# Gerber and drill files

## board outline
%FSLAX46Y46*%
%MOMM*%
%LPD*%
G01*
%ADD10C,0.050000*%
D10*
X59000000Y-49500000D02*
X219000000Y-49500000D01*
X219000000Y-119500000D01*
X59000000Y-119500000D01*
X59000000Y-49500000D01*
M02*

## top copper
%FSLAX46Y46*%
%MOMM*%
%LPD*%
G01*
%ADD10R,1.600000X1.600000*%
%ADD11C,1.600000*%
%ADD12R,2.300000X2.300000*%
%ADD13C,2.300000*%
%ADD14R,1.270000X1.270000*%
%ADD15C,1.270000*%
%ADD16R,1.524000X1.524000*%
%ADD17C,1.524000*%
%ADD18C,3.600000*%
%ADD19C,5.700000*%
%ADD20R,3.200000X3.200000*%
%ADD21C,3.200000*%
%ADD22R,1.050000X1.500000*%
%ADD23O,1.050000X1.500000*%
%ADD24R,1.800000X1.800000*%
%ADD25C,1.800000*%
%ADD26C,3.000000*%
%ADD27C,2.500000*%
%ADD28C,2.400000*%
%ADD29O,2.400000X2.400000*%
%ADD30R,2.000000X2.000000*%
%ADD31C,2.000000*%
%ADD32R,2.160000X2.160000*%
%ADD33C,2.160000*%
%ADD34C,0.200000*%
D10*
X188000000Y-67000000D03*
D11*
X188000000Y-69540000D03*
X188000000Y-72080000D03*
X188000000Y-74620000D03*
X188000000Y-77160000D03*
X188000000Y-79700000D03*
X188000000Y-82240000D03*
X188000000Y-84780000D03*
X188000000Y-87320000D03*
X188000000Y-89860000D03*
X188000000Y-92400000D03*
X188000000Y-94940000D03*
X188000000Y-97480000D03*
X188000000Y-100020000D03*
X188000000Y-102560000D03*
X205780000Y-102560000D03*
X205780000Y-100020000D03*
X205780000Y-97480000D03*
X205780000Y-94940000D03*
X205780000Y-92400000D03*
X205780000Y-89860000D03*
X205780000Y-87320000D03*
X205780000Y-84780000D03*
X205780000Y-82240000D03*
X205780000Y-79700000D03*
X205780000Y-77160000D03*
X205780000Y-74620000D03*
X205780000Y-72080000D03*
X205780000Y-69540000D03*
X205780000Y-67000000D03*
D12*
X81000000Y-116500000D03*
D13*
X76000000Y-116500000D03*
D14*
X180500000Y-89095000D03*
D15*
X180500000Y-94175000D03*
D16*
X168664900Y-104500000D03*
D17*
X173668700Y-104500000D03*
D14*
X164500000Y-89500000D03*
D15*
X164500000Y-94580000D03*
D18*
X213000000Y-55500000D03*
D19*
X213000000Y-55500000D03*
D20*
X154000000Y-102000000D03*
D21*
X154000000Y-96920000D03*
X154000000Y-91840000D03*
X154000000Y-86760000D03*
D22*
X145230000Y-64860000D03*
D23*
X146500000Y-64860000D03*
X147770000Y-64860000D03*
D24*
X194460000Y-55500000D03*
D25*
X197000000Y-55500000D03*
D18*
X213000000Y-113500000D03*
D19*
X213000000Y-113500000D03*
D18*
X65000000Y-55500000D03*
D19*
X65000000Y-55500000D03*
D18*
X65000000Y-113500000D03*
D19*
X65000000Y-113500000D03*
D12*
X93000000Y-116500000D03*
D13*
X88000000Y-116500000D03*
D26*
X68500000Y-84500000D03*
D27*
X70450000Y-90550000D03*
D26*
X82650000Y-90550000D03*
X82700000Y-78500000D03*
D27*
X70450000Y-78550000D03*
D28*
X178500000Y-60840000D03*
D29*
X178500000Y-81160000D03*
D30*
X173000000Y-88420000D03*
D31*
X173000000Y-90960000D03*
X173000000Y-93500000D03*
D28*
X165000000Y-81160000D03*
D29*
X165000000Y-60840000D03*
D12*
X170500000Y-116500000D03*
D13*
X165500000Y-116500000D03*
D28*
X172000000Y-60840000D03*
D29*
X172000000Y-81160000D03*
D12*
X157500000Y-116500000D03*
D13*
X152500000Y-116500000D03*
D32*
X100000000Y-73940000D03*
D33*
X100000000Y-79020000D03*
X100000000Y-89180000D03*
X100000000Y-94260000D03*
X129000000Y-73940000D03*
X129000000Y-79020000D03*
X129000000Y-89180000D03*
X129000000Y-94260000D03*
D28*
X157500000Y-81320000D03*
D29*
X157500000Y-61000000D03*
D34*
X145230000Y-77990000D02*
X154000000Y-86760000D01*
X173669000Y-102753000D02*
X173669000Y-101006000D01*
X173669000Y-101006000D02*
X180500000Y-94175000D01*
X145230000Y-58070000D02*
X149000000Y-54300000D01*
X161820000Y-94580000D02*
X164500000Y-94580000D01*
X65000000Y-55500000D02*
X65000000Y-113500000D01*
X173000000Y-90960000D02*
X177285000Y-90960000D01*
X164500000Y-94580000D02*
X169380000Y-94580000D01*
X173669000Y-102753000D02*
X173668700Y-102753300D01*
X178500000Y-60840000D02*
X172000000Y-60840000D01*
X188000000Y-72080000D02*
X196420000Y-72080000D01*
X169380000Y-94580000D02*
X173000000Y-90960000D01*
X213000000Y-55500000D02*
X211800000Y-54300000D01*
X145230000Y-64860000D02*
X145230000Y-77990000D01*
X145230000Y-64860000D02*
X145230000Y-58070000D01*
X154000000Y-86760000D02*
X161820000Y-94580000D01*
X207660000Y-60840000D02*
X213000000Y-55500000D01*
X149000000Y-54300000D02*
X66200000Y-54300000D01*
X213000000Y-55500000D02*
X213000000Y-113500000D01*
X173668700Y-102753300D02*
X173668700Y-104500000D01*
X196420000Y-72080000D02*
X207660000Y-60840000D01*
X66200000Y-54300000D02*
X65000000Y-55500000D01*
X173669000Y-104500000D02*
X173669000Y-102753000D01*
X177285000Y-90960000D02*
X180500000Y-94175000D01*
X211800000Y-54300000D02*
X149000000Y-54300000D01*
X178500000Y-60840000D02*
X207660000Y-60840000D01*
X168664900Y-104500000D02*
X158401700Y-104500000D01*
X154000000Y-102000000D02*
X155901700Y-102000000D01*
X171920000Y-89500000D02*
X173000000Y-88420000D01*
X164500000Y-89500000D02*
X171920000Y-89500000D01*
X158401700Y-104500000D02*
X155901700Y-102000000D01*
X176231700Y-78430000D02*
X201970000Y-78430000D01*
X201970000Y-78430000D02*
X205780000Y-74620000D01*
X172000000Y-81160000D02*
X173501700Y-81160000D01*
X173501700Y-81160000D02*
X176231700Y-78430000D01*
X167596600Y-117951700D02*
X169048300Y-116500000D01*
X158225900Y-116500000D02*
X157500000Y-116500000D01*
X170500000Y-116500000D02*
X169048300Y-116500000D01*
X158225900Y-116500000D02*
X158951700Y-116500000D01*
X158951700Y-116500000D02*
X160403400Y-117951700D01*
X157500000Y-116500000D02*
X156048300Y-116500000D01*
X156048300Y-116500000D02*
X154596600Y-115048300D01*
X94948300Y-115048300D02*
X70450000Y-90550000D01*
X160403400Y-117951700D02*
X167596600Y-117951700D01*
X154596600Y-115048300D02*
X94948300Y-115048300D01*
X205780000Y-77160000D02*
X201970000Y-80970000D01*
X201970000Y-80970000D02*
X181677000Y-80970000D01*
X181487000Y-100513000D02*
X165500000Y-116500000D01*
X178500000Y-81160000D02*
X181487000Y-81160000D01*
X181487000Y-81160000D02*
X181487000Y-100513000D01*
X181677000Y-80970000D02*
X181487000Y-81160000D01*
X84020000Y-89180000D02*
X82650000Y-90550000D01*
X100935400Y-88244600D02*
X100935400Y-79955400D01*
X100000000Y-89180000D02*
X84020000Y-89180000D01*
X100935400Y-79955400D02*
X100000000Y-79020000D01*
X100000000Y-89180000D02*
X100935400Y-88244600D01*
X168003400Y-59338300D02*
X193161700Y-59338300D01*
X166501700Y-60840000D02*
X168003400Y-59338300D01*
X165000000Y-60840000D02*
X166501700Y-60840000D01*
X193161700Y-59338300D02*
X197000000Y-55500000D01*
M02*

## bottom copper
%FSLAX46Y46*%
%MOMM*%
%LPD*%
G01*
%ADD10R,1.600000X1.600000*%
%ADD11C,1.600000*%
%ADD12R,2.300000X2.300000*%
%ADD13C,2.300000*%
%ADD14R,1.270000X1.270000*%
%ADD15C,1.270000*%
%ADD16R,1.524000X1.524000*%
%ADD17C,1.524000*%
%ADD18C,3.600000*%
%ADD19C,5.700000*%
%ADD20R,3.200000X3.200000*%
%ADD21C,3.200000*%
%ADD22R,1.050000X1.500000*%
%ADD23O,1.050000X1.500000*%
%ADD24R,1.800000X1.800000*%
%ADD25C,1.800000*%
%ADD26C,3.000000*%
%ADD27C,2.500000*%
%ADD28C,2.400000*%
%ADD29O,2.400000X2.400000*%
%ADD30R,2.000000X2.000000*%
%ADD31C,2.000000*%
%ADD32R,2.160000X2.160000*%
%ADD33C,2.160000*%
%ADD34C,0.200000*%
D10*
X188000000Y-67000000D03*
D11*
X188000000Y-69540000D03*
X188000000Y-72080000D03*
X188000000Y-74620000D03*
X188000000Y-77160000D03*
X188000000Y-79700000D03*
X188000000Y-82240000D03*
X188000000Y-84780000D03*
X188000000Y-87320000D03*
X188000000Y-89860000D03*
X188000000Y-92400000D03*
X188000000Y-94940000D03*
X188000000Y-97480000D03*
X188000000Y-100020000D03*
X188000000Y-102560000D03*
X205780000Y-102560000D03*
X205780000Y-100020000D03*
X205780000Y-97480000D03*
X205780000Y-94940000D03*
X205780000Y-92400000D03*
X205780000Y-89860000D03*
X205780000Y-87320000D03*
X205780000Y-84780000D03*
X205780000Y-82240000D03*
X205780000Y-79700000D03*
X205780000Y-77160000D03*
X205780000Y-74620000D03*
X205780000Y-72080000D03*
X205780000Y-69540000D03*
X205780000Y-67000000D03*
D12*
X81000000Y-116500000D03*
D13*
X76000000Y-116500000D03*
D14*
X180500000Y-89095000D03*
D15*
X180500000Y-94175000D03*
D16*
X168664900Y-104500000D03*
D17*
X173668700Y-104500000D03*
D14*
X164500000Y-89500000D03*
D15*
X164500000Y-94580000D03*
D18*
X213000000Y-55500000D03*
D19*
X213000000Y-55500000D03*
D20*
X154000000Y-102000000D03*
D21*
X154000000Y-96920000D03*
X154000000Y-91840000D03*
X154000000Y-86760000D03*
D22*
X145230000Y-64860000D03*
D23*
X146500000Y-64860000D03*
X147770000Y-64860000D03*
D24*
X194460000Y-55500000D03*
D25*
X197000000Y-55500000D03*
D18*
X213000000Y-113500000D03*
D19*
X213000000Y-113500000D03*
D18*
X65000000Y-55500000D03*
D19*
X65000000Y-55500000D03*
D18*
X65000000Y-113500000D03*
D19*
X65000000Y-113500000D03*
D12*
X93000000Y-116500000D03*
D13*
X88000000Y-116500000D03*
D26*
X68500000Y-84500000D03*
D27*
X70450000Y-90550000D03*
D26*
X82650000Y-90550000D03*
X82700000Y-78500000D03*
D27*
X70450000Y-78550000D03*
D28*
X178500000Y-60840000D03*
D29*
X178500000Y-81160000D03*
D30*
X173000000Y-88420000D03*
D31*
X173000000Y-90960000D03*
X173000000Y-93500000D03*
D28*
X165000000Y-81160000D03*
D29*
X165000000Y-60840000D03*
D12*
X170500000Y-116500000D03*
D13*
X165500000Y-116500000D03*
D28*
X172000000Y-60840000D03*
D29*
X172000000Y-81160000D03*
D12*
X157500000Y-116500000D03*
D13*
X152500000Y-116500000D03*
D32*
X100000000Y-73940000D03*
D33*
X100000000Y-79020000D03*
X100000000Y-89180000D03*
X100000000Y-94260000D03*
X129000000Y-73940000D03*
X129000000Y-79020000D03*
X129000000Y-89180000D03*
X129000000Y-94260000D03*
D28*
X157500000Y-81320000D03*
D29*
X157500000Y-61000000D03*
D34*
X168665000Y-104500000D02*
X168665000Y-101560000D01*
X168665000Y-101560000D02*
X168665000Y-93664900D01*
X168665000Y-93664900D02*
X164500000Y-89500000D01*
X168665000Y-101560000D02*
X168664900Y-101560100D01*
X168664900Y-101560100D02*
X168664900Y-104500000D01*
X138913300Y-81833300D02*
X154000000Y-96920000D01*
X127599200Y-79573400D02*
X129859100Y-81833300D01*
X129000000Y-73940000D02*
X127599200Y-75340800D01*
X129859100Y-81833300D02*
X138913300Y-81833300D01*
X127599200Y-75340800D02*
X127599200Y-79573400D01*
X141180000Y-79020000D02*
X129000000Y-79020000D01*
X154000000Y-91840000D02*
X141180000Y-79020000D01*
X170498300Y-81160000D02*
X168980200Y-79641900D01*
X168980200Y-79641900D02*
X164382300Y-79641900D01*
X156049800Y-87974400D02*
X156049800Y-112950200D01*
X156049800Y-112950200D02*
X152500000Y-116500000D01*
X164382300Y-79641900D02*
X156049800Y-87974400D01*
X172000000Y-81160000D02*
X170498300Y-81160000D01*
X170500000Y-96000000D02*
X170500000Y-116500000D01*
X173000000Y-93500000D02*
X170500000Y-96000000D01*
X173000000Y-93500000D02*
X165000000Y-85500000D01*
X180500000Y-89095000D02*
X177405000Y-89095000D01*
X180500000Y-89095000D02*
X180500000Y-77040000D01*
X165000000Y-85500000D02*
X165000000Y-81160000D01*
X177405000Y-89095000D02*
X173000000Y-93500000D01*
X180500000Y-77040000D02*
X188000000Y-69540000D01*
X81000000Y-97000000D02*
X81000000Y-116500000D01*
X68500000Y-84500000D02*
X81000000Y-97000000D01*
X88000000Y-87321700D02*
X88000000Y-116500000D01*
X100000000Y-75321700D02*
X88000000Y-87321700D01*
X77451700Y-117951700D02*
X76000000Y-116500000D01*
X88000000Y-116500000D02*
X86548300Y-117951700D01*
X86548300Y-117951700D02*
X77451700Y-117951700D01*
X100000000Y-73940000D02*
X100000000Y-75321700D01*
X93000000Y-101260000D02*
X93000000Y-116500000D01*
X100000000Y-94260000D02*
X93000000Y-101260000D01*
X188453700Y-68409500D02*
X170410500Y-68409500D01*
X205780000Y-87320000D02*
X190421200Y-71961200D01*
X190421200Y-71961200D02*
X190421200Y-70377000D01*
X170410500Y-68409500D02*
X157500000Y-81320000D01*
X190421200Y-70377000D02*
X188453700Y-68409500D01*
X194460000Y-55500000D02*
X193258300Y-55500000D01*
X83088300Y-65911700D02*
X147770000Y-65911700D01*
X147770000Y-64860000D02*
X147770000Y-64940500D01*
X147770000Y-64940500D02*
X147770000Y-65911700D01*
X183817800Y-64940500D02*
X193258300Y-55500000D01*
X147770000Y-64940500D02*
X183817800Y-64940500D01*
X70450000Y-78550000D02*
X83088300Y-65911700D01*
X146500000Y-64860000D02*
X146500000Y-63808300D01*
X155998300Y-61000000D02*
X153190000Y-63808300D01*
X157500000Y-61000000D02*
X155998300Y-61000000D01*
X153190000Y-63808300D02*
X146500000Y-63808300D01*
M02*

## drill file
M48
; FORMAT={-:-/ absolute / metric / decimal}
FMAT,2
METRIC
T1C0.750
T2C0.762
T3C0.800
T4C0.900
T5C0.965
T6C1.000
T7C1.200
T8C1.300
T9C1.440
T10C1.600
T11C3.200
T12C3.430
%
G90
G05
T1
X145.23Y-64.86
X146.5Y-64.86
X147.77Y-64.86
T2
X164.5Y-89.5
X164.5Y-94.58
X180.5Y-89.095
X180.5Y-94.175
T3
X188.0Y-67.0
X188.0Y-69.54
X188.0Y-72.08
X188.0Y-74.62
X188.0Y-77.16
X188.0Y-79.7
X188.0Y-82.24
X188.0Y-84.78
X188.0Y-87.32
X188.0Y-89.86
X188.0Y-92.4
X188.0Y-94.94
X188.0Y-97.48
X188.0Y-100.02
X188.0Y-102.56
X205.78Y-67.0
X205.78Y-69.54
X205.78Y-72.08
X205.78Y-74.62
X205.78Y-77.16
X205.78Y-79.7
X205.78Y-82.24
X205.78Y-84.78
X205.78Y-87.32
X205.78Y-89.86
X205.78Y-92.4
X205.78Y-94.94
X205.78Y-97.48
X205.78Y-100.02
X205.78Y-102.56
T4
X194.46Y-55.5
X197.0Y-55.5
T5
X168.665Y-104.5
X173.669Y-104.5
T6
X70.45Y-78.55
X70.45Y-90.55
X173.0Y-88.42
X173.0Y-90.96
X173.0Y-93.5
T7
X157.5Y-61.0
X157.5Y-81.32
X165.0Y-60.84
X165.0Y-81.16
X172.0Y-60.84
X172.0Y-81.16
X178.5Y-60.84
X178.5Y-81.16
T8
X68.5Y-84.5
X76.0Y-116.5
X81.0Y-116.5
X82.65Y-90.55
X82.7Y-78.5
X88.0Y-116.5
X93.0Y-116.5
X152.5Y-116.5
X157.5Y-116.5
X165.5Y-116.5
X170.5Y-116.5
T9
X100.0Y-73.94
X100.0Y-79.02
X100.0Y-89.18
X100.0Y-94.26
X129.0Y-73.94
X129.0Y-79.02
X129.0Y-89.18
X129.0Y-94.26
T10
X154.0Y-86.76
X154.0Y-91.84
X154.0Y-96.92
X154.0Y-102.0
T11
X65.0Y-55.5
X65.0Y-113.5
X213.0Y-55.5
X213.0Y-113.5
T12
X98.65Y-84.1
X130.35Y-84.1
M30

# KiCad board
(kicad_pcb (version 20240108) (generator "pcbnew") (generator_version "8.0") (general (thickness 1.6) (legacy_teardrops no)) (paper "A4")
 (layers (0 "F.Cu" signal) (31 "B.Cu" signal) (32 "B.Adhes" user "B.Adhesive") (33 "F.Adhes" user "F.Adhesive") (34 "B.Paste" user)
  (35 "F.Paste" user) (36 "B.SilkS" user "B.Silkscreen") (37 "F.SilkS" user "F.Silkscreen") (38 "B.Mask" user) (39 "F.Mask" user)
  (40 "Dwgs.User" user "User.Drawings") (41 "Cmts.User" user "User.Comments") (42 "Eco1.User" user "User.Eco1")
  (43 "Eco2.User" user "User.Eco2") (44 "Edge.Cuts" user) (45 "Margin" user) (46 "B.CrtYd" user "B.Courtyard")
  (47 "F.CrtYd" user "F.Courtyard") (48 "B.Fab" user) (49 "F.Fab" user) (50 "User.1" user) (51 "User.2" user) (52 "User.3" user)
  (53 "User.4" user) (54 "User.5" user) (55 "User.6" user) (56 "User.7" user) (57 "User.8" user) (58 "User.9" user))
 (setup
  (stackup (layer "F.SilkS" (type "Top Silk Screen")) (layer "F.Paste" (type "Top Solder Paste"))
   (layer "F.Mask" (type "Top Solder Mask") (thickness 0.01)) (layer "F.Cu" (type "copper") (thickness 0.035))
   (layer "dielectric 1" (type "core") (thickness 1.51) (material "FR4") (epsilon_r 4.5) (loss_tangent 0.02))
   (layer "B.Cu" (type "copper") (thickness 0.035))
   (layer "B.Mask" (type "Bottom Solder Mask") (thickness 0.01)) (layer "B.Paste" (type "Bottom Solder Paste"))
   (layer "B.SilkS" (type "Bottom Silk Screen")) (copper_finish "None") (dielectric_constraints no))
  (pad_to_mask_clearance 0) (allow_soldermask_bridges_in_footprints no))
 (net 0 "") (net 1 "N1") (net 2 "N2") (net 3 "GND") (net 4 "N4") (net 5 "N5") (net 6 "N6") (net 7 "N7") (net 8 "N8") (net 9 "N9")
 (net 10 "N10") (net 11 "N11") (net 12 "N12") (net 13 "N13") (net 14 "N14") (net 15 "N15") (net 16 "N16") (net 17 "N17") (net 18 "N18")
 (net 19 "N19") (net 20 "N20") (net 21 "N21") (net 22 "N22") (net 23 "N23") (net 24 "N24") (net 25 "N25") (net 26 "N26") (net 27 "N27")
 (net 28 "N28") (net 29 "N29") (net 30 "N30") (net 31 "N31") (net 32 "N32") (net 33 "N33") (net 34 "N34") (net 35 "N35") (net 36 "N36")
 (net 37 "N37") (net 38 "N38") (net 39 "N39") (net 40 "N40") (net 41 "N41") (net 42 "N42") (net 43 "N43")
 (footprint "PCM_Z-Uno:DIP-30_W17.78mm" (layer "F.Cu") (at 188 67)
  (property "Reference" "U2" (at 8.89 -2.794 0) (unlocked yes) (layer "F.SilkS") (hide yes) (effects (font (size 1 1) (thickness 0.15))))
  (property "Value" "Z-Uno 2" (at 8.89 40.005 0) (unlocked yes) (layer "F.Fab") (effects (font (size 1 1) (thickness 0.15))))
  (pad "1" thru_hole rect (at 0 0) (size 1.6 1.6) (drill 0.8) (layers "*.Cu" "*.Mask") (remove_unused_layers no) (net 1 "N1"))
  (pad "2" thru_hole circle (at 0 2.54) (size 1.6 1.6) (drill 0.8) (layers "*.Cu" "*.Mask") (remove_unused_layers no) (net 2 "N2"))
  (pad "3" thru_hole circle (at 0 5.08) (size 1.6 1.6) (drill 0.8) (layers "*.Cu" "*.Mask") (remove_unused_layers no) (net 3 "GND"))
  (pad "4" thru_hole circle (at 0 7.62) (size 1.6 1.6) (drill 0.8) (layers "*.Cu" "*.Mask") (remove_unused_layers no) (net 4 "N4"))
  (pad "5" thru_hole circle (at 0 10.16) (size 1.6 1.6) (drill 0.8) (layers "*.Cu" "*.Mask") (remove_unused_layers no) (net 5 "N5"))
  (pad "6" thru_hole circle (at 0 12.7) (size 1.6 1.6) (drill 0.8) (layers "*.Cu" "*.Mask") (remove_unused_layers no) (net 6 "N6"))
  (pad "7" thru_hole circle (at 0 15.24) (size 1.6 1.6) (drill 0.8) (layers "*.Cu" "*.Mask") (remove_unused_layers no) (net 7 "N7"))
  (pad "8" thru_hole circle (at 0 17.78) (size 1.6 1.6) (drill 0.8) (layers "*.Cu" "*.Mask") (remove_unused_layers no) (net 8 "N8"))
  (pad "9" thru_hole circle (at 0 20.32) (size 1.6 1.6) (drill 0.8) (layers "*.Cu" "*.Mask") (remove_unused_layers no) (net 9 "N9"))
  (pad "10" thru_hole circle (at 0 22.86) (size 1.6 1.6) (drill 0.8) (layers "*.Cu" "*.Mask") (remove_unused_layers no) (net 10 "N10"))
  (pad "11" thru_hole circle (at 0 25.4) (size 1.6 1.6) (drill 0.8) (layers "*.Cu" "*.Mask") (remove_unused_layers no) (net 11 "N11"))
  (pad "12" thru_hole circle (at 0 27.94) (size 1.6 1.6) (drill 0.8) (layers "*.Cu" "*.Mask") (remove_unused_layers no) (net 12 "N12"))
  (pad "13" thru_hole circle (at 0 30.48) (size 1.6 1.6) (drill 0.8) (layers "*.Cu" "*.Mask") (remove_unused_layers no) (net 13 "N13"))
  (pad "14" thru_hole circle (at 0 33.02) (size 1.6 1.6) (drill 0.8) (layers "*.Cu" "*.Mask") (remove_unused_layers no) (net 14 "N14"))
  (pad "15" thru_hole circle (at 0 35.56) (size 1.6 1.6) (drill 0.8) (layers "*.Cu" "*.Mask") (remove_unused_layers no) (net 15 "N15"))
  (pad "16" thru_hole circle (at 17.78 35.56) (size 1.6 1.6) (drill 0.8) (layers "*.Cu" "*.Mask") (remove_unused_layers no) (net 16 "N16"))
  (pad "17" thru_hole circle (at 17.78 33.02) (size 1.6 1.6) (drill 0.8) (layers "*.Cu" "*.Mask") (remove_unused_layers no) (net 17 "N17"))
  (pad "18" thru_hole circle (at 17.78 30.48) (size 1.6 1.6) (drill 0.8) (layers "*.Cu" "*.Mask") (remove_unused_layers no) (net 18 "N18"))
  (pad "19" thru_hole circle (at 17.78 27.94) (size 1.6 1.6) (drill 0.8) (layers "*.Cu" "*.Mask") (remove_unused_layers no) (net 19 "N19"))
  (pad "20" thru_hole circle (at 17.78 25.4) (size 1.6 1.6) (drill 0.8) (layers "*.Cu" "*.Mask") (remove_unused_layers no) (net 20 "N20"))
  (pad "21" thru_hole circle (at 17.78 22.86) (size 1.6 1.6) (drill 0.8) (layers "*.Cu" "*.Mask") (remove_unused_layers no) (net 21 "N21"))
  (pad "22" thru_hole circle (at 17.78 20.32) (size 1.6 1.6) (drill 0.8) (layers "*.Cu" "*.Mask") (remove_unused_layers no) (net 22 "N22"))
  (pad "23" thru_hole circle (at 17.78 17.78) (size 1.6 1.6) (drill 0.8) (layers "*.Cu" "*.Mask") (remove_unused_layers no) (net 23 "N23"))
  (pad "24" thru_hole circle (at 17.78 15.24) (size 1.6 1.6) (drill 0.8) (layers "*.Cu" "*.Mask") (remove_unused_layers no) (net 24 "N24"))
  (pad "25" thru_hole circle (at 17.78 12.7) (size 1.6 1.6) (drill 0.8) (layers "*.Cu" "*.Mask") (remove_unused_layers no) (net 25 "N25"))
  (pad "26" thru_hole circle (at 17.78 10.16) (size 1.6 1.6) (drill 0.8) (layers "*.Cu" "*.Mask") (remove_unused_layers no) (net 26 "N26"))
  (pad "27" thru_hole circle (at 17.78 7.62) (size 1.6 1.6) (drill 0.8) (layers "*.Cu" "*.Mask") (remove_unused_layers no) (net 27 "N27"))
  (pad "28" thru_hole circle (at 17.78 5.08) (size 1.6 1.6) (drill 0.8) (layers "*.Cu" "*.Mask") (remove_unused_layers no) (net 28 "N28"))
  (pad "29" thru_hole circle (at 17.78 2.54) (size 1.6 1.6) (drill 0.8) (layers "*.Cu" "*.Mask") (remove_unused_layers no) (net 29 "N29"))
  (pad "30" thru_hole circle (at 17.78 0) (size 1.6 1.6) (drill 0.8) (layers "*.Cu" "*.Mask") (remove_unused_layers no) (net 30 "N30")))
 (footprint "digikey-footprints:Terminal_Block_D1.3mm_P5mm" (layer "F.Cu") (at 81 116.5 180)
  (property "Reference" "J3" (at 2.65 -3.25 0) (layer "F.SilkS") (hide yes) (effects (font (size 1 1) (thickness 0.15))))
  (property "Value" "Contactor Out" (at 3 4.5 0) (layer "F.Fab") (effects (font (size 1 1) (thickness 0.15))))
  (pad "1" thru_hole rect (at 0 0 180) (size 2.3 2.3) (drill 1.3) (layers "*.Cu" "*.Mask") (remove_unused_layers no) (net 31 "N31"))
  (pad "2" thru_hole circle (at 5 0 180) (size 2.3 2.3) (drill 1.3) (layers "*.Cu" "*.Mask") (remove_unused_layers no) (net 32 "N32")))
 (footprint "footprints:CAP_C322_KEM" (layer "F.Cu") (at 180.5 89.095 -90)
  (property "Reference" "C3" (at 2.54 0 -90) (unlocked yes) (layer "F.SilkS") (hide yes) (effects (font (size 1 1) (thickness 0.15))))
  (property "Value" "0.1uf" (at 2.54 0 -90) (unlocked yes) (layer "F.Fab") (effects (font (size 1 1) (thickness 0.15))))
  (pad "1" thru_hole rect (at 0 0 270) (size 1.27 1.27) (drill 0.762) (layers "*.Cu" "*.Mask") (remove_unused_layers no) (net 2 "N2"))
  (pad "2" thru_hole circle (at 5.08 0 270) (size 1.27 1.27) (drill 0.762) (layers "*.Cu" "*.Mask") (remove_unused_layers no) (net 3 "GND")))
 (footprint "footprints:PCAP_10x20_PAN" (layer "F.Cu") (at 168.6649 104.5)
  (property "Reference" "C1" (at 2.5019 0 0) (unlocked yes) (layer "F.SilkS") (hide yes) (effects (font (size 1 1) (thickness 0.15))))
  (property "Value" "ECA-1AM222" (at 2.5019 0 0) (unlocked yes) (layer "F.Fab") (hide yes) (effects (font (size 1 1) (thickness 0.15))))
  (pad "1" thru_hole rect (at 0 0) (size 1.524 1.524) (drill 0.9652) (layers "*.Cu" "*.Mask") (remove_unused_layers no) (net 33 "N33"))
  (pad "2" thru_hole circle (at 5.0038 0) (size 1.524 1.524) (drill 0.9652) (layers "*.Cu" "*.Mask") (remove_unused_layers no) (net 3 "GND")))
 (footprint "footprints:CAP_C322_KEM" (layer "F.Cu") (at 164.5 89.5 -90)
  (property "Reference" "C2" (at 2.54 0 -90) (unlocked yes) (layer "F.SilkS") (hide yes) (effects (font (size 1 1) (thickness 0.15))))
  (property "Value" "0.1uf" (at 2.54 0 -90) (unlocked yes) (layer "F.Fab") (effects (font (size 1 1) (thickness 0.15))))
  (pad "1" thru_hole rect (at 0 0 270) (size 1.27 1.27) (drill 0.762) (layers "*.Cu" "*.Mask") (remove_unused_layers no) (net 33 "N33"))
  (pad "2" thru_hole circle (at 5.08 0 270) (size 1.27 1.27) (drill 0.762) (layers "*.Cu" "*.Mask") (remove_unused_layers no) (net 3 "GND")))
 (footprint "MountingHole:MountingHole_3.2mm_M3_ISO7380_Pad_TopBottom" (layer "F.Cu") (at 213 55.5)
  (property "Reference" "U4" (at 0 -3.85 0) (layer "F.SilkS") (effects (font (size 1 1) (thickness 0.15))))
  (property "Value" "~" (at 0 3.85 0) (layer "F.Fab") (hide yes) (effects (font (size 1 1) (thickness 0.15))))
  (pad "1" thru_hole circle (at 0 0) (size 3.6 3.6) (drill 3.2) (layers "*.Cu" "*.Mask") (remove_unused_layers no) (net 3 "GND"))
  (pad "1" connect circle (at 0 0) (size 5.7 5.7) (layers "F.Cu" "F.Mask") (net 3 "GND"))
  (pad "1" connect circle (at 0 0) (size 5.7 5.7) (layers "B.Cu" "B.Mask") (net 3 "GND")))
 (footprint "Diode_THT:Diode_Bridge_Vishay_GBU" (layer "F.Cu") (at 154 102 90)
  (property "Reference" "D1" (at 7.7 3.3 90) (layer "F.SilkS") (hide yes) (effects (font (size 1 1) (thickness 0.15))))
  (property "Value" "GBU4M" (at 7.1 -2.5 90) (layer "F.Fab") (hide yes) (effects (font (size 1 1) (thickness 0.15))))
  (pad "1" thru_hole rect (at 0 0 90) (size 3.2 3.2) (drill 1.6) (layers "*.Cu" "*.Mask") (remove_unused_layers no) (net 33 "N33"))
  (pad "2" thru_hole circle (at 5.08 0 90) (size 3.2 3.2) (drill 1.6) (layers "*.Cu" "*.Mask") (remove_unused_layers no) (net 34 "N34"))
  (pad "3" thru_hole circle (at 10.16 0 90) (size 3.2 3.2) (drill 1.6) (layers "*.Cu" "*.Mask") (remove_unused_layers no) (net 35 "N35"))
  (pad "4" thru_hole circle (at 15.24 0 90) (size 3.2 3.2) (drill 1.6) (layers "*.Cu" "*.Mask") (remove_unused_layers no) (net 3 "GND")))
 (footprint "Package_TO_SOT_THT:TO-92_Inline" (layer "F.Cu") (at 145.23 64.86)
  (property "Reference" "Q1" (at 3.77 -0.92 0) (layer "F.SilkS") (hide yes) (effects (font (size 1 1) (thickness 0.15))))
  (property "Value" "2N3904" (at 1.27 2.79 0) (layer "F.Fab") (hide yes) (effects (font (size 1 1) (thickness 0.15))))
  (pad "1" thru_hole rect (at 0 0) (size 1.05 1.5) (drill 0.75) (layers "*.Cu" "*.Mask") (remove_unused_layers no) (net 3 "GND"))
  (pad "2" thru_hole oval (at 1.27 0) (size 1.05 1.5) (drill 0.75) (layers "*.Cu" "*.Mask") (remove_unused_layers no) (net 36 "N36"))
  (pad "3" thru_hole oval (at 2.54 0) (size 1.05 1.5) (drill 0.75) (layers "*.Cu" "*.Mask") (remove_unused_layers no) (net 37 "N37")))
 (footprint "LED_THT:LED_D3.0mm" (layer "F.Cu") (at 194.46 55.5)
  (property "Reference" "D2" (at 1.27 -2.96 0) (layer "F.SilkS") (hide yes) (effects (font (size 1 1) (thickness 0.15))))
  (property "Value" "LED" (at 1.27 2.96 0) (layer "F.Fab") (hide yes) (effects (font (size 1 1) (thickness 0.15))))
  (pad "1" thru_hole rect (at 0 0) (size 1.8 1.8) (drill 0.9) (layers "*.Cu" "*.Mask") (remove_unused_layers no) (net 37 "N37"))
  (pad "2" thru_hole circle (at 2.54 0) (size 1.8 1.8) (drill 0.9) (layers "*.Cu" "*.Mask") (remove_unused_layers no) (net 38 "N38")))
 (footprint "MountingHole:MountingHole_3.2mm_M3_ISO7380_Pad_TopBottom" (layer "F.Cu") (at 213 113.5)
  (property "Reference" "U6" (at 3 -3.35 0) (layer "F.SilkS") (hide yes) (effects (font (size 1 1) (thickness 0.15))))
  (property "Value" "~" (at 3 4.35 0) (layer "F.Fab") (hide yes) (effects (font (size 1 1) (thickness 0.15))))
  (pad "1" thru_hole circle (at 0 0) (size 3.6 3.6) (drill 3.2) (layers "*.Cu" "*.Mask") (remove_unused_layers no) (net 3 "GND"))
  (pad "1" connect circle (at 0 0) (size 5.7 5.7) (layers "F.Cu" "F.Mask") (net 3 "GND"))
  (pad "1" connect circle (at 0 0) (size 5.7 5.7) (layers "B.Cu" "B.Mask") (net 3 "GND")))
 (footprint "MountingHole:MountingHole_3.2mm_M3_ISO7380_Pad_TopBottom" (layer "F.Cu") (at 65 55.5)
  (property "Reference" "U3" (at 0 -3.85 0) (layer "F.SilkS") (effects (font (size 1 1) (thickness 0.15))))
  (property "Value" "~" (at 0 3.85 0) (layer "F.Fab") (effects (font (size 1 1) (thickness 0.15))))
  (pad "1" thru_hole circle (at 0 0) (size 3.6 3.6) (drill 3.2) (layers "*.Cu" "*.Mask") (remove_unused_layers no) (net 3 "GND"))
  (pad "1" connect circle (at 0 0) (size 5.7 5.7) (layers "F.Cu" "F.Mask") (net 3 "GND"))
  (pad "1" connect circle (at 0 0) (size 5.7 5.7) (layers "B.Cu" "B.Mask") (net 3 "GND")))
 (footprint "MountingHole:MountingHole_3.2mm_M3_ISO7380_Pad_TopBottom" (layer "F.Cu") (at 65 113.5)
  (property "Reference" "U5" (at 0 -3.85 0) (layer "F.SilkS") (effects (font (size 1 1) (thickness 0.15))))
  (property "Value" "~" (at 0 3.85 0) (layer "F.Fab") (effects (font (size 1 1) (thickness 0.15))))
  (pad "1" thru_hole circle (at 0 0) (size 3.6 3.6) (drill 3.2) (layers "*.Cu" "*.Mask") (remove_unused_layers no) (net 3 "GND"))
  (pad "1" connect circle (at 0 0) (size 5.7 5.7) (layers "F.Cu" "F.Mask") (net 3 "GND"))
  (pad "1" connect circle (at 0 0) (size 5.7 5.7) (layers "B.Cu" "B.Mask") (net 3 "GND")))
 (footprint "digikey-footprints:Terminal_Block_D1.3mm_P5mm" (layer "F.Cu") (at 93 116.5 180)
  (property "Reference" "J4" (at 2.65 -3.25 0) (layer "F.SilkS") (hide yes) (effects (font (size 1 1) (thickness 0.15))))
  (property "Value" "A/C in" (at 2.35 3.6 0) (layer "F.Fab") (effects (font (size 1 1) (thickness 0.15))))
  (pad "1" thru_hole rect (at 0 0 180) (size 2.3 2.3) (drill 1.3) (layers "*.Cu" "*.Mask") (remove_unused_layers no) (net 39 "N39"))
  (pad "2" thru_hole circle (at 5 0 180) (size 2.3 2.3) (drill 1.3) (layers "*.Cu" "*.Mask") (remove_unused_layers no) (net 32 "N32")))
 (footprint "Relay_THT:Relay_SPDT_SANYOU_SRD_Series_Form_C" (layer "F.Cu") (at 68.5 84.5)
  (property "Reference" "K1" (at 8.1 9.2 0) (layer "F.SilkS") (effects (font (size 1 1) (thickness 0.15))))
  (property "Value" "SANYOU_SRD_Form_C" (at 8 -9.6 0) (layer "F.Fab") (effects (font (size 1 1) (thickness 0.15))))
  (pad "1" thru_hole circle (at 0 0 90) (size 3 3) (drill 1.3) (layers "*.Cu" "*.Mask") (remove_unused_layers no) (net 31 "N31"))
  (pad "2" thru_hole circle (at 1.95 6.05 90) (size 2.5 2.5) (drill 1) (layers "*.Cu" "*.Mask") (remove_unused_layers no) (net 2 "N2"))
  (pad "3" thru_hole circle (at 14.15 6.05 90) (size 3 3) (drill 1.3) (layers "*.Cu" "*.Mask") (remove_unused_layers no) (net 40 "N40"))
  (pad "4" thru_hole circle (at 14.2 -6 90) (size 3 3) (drill 1.3) (layers "*.Cu" "*.Mask") (remove_unused_layers no) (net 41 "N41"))
  (pad "5" thru_hole circle (at 1.95 -5.95 90) (size 2.5 2.5) (drill 1) (layers "*.Cu" "*.Mask") (remove_unused_layers no) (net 37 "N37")))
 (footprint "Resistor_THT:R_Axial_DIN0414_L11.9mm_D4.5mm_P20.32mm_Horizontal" (layer "F.Cu") (at 178.5 60.84 -90)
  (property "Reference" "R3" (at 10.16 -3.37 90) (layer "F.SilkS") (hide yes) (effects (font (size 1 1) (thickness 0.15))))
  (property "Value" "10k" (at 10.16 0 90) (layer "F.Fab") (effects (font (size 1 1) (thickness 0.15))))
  (pad "1" thru_hole circle (at 0 0 270) (size 2.4 2.4) (drill 1.2) (layers "*.Cu" "*.Mask") (remove_unused_layers no) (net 3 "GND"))
  (pad "2" thru_hole oval (at 20.32 0 270) (size 2.4 2.4) (drill 1.2) (layers "*.Cu" "*.Mask") (remove_unused_layers no) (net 26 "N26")))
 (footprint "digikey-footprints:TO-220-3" (layer "F.Cu") (at 173 88.42 -90)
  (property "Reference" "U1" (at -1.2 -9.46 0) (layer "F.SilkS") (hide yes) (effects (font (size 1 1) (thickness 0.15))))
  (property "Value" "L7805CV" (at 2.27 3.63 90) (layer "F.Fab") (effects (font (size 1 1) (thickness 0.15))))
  (pad "1" thru_hole rect (at 0 0 270) (size 2 2) (drill 1) (layers "*.Cu" "*.Mask") (remove_unused_layers no) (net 33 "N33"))
  (pad "2" thru_hole circle (at 2.54 0 270) (size 2 2) (drill 1) (layers "*.Cu" "*.Mask") (remove_unused_layers no) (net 3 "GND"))
  (pad "3" thru_hole circle (at 5.08 0 270) (size 2 2) (drill 1) (layers "*.Cu" "*.Mask") (remove_unused_layers no) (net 2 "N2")))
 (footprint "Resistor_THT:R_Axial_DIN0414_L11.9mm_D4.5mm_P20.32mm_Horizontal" (layer "F.Cu") (at 165 81.16 90)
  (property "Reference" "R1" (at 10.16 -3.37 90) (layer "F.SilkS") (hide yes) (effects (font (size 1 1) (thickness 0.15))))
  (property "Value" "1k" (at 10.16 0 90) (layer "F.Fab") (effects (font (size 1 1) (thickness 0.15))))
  (pad "1" thru_hole circle (at 0 0 90) (size 2.4 2.4) (drill 1.2) (layers "*.Cu" "*.Mask") (remove_unused_layers no) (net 2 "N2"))
  (pad "2" thru_hole oval (at 20.32 0 90) (size 2.4 2.4) (drill 1.2) (layers "*.Cu" "*.Mask") (remove_unused_layers no) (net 38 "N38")))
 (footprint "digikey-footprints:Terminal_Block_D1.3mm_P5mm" (layer "F.Cu") (at 170.5 116.5 180)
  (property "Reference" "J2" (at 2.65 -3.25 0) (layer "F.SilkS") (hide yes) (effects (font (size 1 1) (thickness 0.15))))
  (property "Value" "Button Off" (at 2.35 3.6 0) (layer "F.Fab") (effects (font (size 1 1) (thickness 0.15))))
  (pad "1" thru_hole rect (at 0 0 180) (size 2.3 2.3) (drill 1.3) (layers "*.Cu" "*.Mask") (remove_unused_layers no) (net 2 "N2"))
  (pad "2" thru_hole circle (at 5 0 180) (size 2.3 2.3) (drill 1.3) (layers "*.Cu" "*.Mask") (remove_unused_layers no) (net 26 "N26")))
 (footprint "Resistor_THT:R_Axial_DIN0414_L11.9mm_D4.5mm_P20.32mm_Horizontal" (layer "F.Cu") (at 172 60.84 -90)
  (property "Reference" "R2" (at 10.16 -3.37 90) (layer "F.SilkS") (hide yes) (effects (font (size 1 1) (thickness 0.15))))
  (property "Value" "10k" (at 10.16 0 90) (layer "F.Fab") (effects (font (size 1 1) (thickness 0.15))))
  (pad "1" thru_hole circle (at 0 0 270) (size 2.4 2.4) (drill 1.2) (layers "*.Cu" "*.Mask") (remove_unused_layers no) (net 3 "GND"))
  (pad "2" thru_hole oval (at 20.32 0 270) (size 2.4 2.4) (drill 1.2) (layers "*.Cu" "*.Mask") (remove_unused_layers no) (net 27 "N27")))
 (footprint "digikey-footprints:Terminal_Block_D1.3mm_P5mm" (layer "F.Cu") (at 157.5 116.5 180)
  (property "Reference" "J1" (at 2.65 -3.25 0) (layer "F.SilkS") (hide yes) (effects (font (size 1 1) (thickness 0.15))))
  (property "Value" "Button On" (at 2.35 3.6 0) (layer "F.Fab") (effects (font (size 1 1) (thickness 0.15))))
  (pad "1" thru_hole rect (at 0 0 180) (size 2.3 2.3) (drill 1.3) (layers "*.Cu" "*.Mask") (remove_unused_layers no) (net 2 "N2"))
  (pad "2" thru_hole circle (at 5 0 180) (size 2.3 2.3) (drill 1.3) (layers "*.Cu" "*.Mask") (remove_unused_layers no) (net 27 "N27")))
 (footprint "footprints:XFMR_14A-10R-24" (layer "F.Cu") (at 114.5 84.1)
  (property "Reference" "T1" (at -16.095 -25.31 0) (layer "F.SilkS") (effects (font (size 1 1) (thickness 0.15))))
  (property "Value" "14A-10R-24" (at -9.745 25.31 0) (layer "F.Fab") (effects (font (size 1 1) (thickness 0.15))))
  (pad "" np_thru_hole circle (at -15.85 0) (size 3.43 3.43) (drill 3.43) (layers "*.Cu" "*.Mask"))
  (pad "" np_thru_hole circle (at 15.85 0) (size 3.43 3.43) (drill 3.43) (layers "*.Cu" "*.Mask"))
  (pad "1" thru_hole rect (at -14.5 -10.16) (size 2.16 2.16) (drill 1.44) (layers "*.Cu" "*.Mask") (remove_unused_layers no) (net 32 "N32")
   (solder_mask_margin 0.102))
  (pad "3" thru_hole circle (at -14.5 -5.08) (size 2.16 2.16) (drill 1.44) (layers "*.Cu" "*.Mask") (remove_unused_layers no) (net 40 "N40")
   (solder_mask_margin 0.102))
  (pad "4" thru_hole circle (at -14.5 5.08) (size 2.16 2.16) (drill 1.44) (layers "*.Cu" "*.Mask") (remove_unused_layers no) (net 40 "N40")
   (solder_mask_margin 0.102))
  (pad "6" thru_hole circle (at -14.5 10.16) (size 2.16 2.16) (drill 1.44) (layers "*.Cu" "*.Mask") (remove_unused_layers no) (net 39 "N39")
   (solder_mask_margin 0.102))
  (pad "7" thru_hole circle (at 14.5 -10.16) (size 2.16 2.16) (drill 1.44) (layers "*.Cu" "*.Mask") (remove_unused_layers no) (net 34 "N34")
   (solder_mask_margin 0.102))
  (pad "9" thru_hole circle (at 14.5 -5.08) (size 2.16 2.16) (drill 1.44) (layers "*.Cu" "*.Mask") (remove_unused_layers no) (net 35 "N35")
   (solder_mask_margin 0.102))
  (pad "10" thru_hole circle (at 14.5 5.08) (size 2.16 2.16) (drill 1.44) (layers "*.Cu" "*.Mask") (remove_unused_layers no) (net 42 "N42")
   (solder_mask_margin 0.102))
  (pad "12" thru_hole circle (at 14.5 10.16) (size 2.16 2.16) (drill 1.44) (layers "*.Cu" "*.Mask") (remove_unused_layers no) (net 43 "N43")
   (solder_mask_margin 0.102)))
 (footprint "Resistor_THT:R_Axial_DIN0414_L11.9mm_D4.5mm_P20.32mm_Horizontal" (layer "F.Cu") (at 157.5 81.32 90)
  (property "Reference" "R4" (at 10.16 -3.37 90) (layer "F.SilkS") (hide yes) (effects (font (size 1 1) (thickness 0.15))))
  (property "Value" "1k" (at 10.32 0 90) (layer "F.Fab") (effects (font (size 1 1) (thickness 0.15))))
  (pad "1" thru_hole circle (at 0 0 90) (size 2.4 2.4) (drill 1.2) (layers "*.Cu" "*.Mask") (remove_unused_layers no) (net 22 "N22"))
  (pad "2" thru_hole oval (at 20.32 0 90) (size 2.4 2.4) (drill 1.2) (layers "*.Cu" "*.Mask") (remove_unused_layers no) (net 36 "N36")))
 (gr_rect (start 59 49.5) (end 219 119.5) (stroke (width 0.05) (type default)) (fill none) (layer "Edge.Cuts"))
 (segment (start 145.23 77.99) (end 154 86.76) (width 0.2) (layer "F.Cu") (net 3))
 (segment (start 173.669 102.753) (end 173.669 101.006) (width 0.2) (layer "F.Cu") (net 3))
 (segment (start 173.669 101.006) (end 180.5 94.175) (width 0.2) (layer "F.Cu") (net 3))
 (segment (start 145.23 58.07) (end 149 54.3) (width 0.2) (layer "F.Cu") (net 3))
 (segment (start 161.82 94.58) (end 164.5 94.58) (width 0.2) (layer "F.Cu") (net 3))
 (segment (start 65 55.5) (end 65 113.5) (width 0.2) (layer "F.Cu") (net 3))
 (segment (start 173 90.96) (end 177.285 90.96) (width 0.2) (layer "F.Cu") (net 3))
 (segment (start 164.5 94.58) (end 169.38 94.58) (width 0.2) (layer "F.Cu") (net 3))
 (segment (start 173.669 102.753) (end 173.6687 102.7533) (width 0.2) (layer "F.Cu") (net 3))
 (segment (start 178.5 60.84) (end 172 60.84) (width 0.2) (layer "F.Cu") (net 3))
 (segment (start 188 72.08) (end 196.42 72.08) (width 0.2) (layer "F.Cu") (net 3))
 (segment (start 169.38 94.58) (end 173 90.96) (width 0.2) (layer "F.Cu") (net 3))
 (segment (start 213 55.5) (end 211.8 54.3) (width 0.2) (layer "F.Cu") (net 3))
 (segment (start 145.23 64.86) (end 145.23 77.99) (width 0.2) (layer "F.Cu") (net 3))
 (segment (start 145.23 64.86) (end 145.23 58.07) (width 0.2) (layer "F.Cu") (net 3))
 (segment (start 154 86.76) (end 161.82 94.58) (width 0.2) (layer "F.Cu") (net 3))
 (segment (start 207.66 60.84) (end 213 55.5) (width 0.2) (layer "F.Cu") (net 3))
 (segment (start 149 54.3) (end 66.2 54.3) (width 0.2) (layer "F.Cu") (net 3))
 (segment (start 213 55.5) (end 213 113.5) (width 0.2) (layer "F.Cu") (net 3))
 (segment (start 173.6687 102.7533) (end 173.6687 104.5) (width 0.2) (layer "F.Cu") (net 3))
 (segment (start 196.42 72.08) (end 207.66 60.84) (width 0.2) (layer "F.Cu") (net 3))
 (segment (start 66.2 54.3) (end 65 55.5) (width 0.2) (layer "F.Cu") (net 3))
 (segment (start 173.669 104.5) (end 173.669 102.753) (width 0.2) (layer "F.Cu") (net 3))
 (segment (start 177.285 90.96) (end 180.5 94.175) (width 0.2) (layer "F.Cu") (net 3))
 (segment (start 211.8 54.3) (end 149 54.3) (width 0.2) (layer "F.Cu") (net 3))
 (segment (start 178.5 60.84) (end 207.66 60.84) (width 0.2) (layer "F.Cu") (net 3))
 (segment (start 168.6649 104.5) (end 158.4017 104.5) (width 0.2) (layer "F.Cu") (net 33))
 (segment (start 154 102) (end 155.9017 102) (width 0.2) (layer "F.Cu") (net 33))
 (segment (start 171.92 89.5) (end 173 88.42) (width 0.2) (layer "F.Cu") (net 33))
 (segment (start 164.5 89.5) (end 171.92 89.5) (width 0.2) (layer "F.Cu") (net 33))
 (segment (start 158.4017 104.5) (end 155.9017 102) (width 0.2) (layer "F.Cu") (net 33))
 (segment (start 168.665 104.5) (end 168.665 101.56) (width 0.2) (layer "B.Cu") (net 33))
 (segment (start 168.665 101.56) (end 168.665 93.6649) (width 0.2) (layer "B.Cu") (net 33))
 (segment (start 168.665 93.6649) (end 164.5 89.5) (width 0.2) (layer "B.Cu") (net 33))
 (segment (start 168.665 101.56) (end 168.6649 101.5601) (width 0.2) (layer "B.Cu") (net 33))
 (segment (start 168.6649 101.5601) (end 168.6649 104.5) (width 0.2) (layer "B.Cu") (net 33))
 (segment (start 138.9133 81.8333) (end 154 96.92) (width 0.2) (layer "B.Cu") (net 34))
 (segment (start 127.5992 79.5734) (end 129.8591 81.8333) (width 0.2) (layer "B.Cu") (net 34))
 (segment (start 129 73.94) (end 127.5992 75.3408) (width 0.2) (layer "B.Cu") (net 34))
 (segment (start 129.8591 81.8333) (end 138.9133 81.8333) (width 0.2) (layer "B.Cu") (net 34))
 (segment (start 127.5992 75.3408) (end 127.5992 79.5734) (width 0.2) (layer "B.Cu") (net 34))
 (segment (start 141.18 79.02) (end 129 79.02) (width 0.2) (layer "B.Cu") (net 35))
 (segment (start 154 91.84) (end 141.18 79.02) (width 0.2) (layer "B.Cu") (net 35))
 (segment (start 176.2317 78.43) (end 201.97 78.43) (width 0.2) (layer "F.Cu") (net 27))
 (segment (start 201.97 78.43) (end 205.78 74.62) (width 0.2) (layer "F.Cu") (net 27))
 (segment (start 172 81.16) (end 173.5017 81.16) (width 0.2) (layer "F.Cu") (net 27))
 (segment (start 173.5017 81.16) (end 176.2317 78.43) (width 0.2) (layer "F.Cu") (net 27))
 (segment (start 170.4983 81.16) (end 168.9802 79.6419) (width 0.2) (layer "B.Cu") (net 27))
 (segment (start 168.9802 79.6419) (end 164.3823 79.6419) (width 0.2) (layer "B.Cu") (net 27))
 (segment (start 156.0498 87.9744) (end 156.0498 112.9502) (width 0.2) (layer "B.Cu") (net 27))
 (segment (start 156.0498 112.9502) (end 152.5 116.5) (width 0.2) (layer "B.Cu") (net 27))
 (segment (start 164.3823 79.6419) (end 156.0498 87.9744) (width 0.2) (layer "B.Cu") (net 27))
 (segment (start 172 81.16) (end 170.4983 81.16) (width 0.2) (layer "B.Cu") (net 27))
 (segment (start 167.5966 117.9517) (end 169.0483 116.5) (width 0.2) (layer "F.Cu") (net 2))
 (segment (start 158.2259 116.5) (end 157.5 116.5) (width 0.2) (layer "F.Cu") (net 2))
 (segment (start 170.5 116.5) (end 169.0483 116.5) (width 0.2) (layer "F.Cu") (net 2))
 (segment (start 158.2259 116.5) (end 158.9517 116.5) (width 0.2) (layer "F.Cu") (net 2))
 (segment (start 158.9517 116.5) (end 160.4034 117.9517) (width 0.2) (layer "F.Cu") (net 2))
 (segment (start 157.5 116.5) (end 156.0483 116.5) (width 0.2) (layer "F.Cu") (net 2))
 (segment (start 156.0483 116.5) (end 154.5966 115.0483) (width 0.2) (layer "F.Cu") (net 2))
 (segment (start 94.9483 115.0483) (end 70.45 90.55) (width 0.2) (layer "F.Cu") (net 2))
 (segment (start 160.4034 117.9517) (end 167.5966 117.9517) (width 0.2) (layer "F.Cu") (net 2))
 (segment (start 154.5966 115.0483) (end 94.9483 115.0483) (width 0.2) (layer "F.Cu") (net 2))
 (segment (start 170.5 96) (end 170.5 116.5) (width 0.2) (layer "B.Cu") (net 2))
 (segment (start 173 93.5) (end 170.5 96) (width 0.2) (layer "B.Cu") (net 2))
 (segment (start 173 93.5) (end 165 85.5) (width 0.2) (layer "B.Cu") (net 2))
 (segment (start 180.5 89.095) (end 177.405 89.095) (width 0.2) (layer "B.Cu") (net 2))
 (segment (start 180.5 89.095) (end 180.5 77.04) (width 0.2) (layer "B.Cu") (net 2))
 (segment (start 165 85.5) (end 165 81.16) (width 0.2) (layer "B.Cu") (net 2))
 (segment (start 177.405 89.095) (end 173 93.5) (width 0.2) (layer "B.Cu") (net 2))
 (segment (start 180.5 77.04) (end 188 69.54) (width 0.2) (layer "B.Cu") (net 2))
 (segment (start 205.78 77.16) (end 201.97 80.97) (width 0.2) (layer "F.Cu") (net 26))
 (segment (start 201.97 80.97) (end 181.677 80.97) (width 0.2) (layer "F.Cu") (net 26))
 (segment (start 181.487 100.513) (end 165.5 116.5) (width 0.2) (layer "F.Cu") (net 26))
 (segment (start 178.5 81.16) (end 181.487 81.16) (width 0.2) (layer "F.Cu") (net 26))
 (segment (start 181.487 81.16) (end 181.487 100.513) (width 0.2) (layer "F.Cu") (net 26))
 (segment (start 181.677 80.97) (end 181.487 81.16) (width 0.2) (layer "F.Cu") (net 26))
 (segment (start 81 97) (end 81 116.5) (width 0.2) (layer "B.Cu") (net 31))
 (segment (start 68.5 84.5) (end 81 97) (width 0.2) (layer "B.Cu") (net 31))
 (segment (start 88 87.3217) (end 88 116.5) (width 0.2) (layer "B.Cu") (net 32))
 (segment (start 100 75.3217) (end 88 87.3217) (width 0.2) (layer "B.Cu") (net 32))
 (segment (start 77.4517 117.9517) (end 76 116.5) (width 0.2) (layer "B.Cu") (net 32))
 (segment (start 88 116.5) (end 86.5483 117.9517) (width 0.2) (layer "B.Cu") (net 32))
 (segment (start 86.5483 117.9517) (end 77.4517 117.9517) (width 0.2) (layer "B.Cu") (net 32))
 (segment (start 100 73.94) (end 100 75.3217) (width 0.2) (layer "B.Cu") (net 32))
 (segment (start 93 101.26) (end 93 116.5) (width 0.2) (layer "B.Cu") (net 39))
 (segment (start 100 94.26) (end 93 101.26) (width 0.2) (layer "B.Cu") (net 39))
 (segment (start 188.4537 68.4095) (end 170.4105 68.4095) (width 0.2) (layer "B.Cu") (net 22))
 (segment (start 205.78 87.32) (end 190.4212 71.9612) (width 0.2) (layer "B.Cu") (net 22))
 (segment (start 190.4212 71.9612) (end 190.4212 70.377) (width 0.2) (layer "B.Cu") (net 22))
 (segment (start 170.4105 68.4095) (end 157.5 81.32) (width 0.2) (layer "B.Cu") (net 22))
 (segment (start 190.4212 70.377) (end 188.4537 68.4095) (width 0.2) (layer "B.Cu") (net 22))
 (segment (start 84.02 89.18) (end 82.65 90.55) (width 0.2) (layer "F.Cu") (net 40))
 (segment (start 100.9354 88.2446) (end 100.9354 79.9554) (width 0.2) (layer "F.Cu") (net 40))
 (segment (start 100 89.18) (end 84.02 89.18) (width 0.2) (layer "F.Cu") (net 40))
 (segment (start 100.9354 79.9554) (end 100 79.02) (width 0.2) (layer "F.Cu") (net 40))
 (segment (start 100 89.18) (end 100.9354 88.2446) (width 0.2) (layer "F.Cu") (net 40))
 (segment (start 194.46 55.5) (end 193.2583 55.5) (width 0.2) (layer "B.Cu") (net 37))
 (segment (start 83.0883 65.9117) (end 147.77 65.9117) (width 0.2) (layer "B.Cu") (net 37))
 (segment (start 147.77 64.86) (end 147.77 64.9405) (width 0.2) (layer "B.Cu") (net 37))
 (segment (start 147.77 64.9405) (end 147.77 65.9117) (width 0.2) (layer "B.Cu") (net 37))
 (segment (start 183.8178 64.9405) (end 193.2583 55.5) (width 0.2) (layer "B.Cu") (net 37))
 (segment (start 147.77 64.9405) (end 183.8178 64.9405) (width 0.2) (layer "B.Cu") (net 37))
 (segment (start 70.45 78.55) (end 83.0883 65.9117) (width 0.2) (layer "B.Cu") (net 37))
 (segment (start 168.0034 59.3383) (end 193.1617 59.3383) (width 0.2) (layer "F.Cu") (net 38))
 (segment (start 166.5017 60.84) (end 168.0034 59.3383) (width 0.2) (layer "F.Cu") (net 38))
 (segment (start 165 60.84) (end 166.5017 60.84) (width 0.2) (layer "F.Cu") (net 38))
 (segment (start 193.1617 59.3383) (end 197 55.5) (width 0.2) (layer "F.Cu") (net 38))
 (segment (start 146.5 64.86) (end 146.5 63.8083) (width 0.2) (layer "B.Cu") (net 36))
 (segment (start 155.9983 61) (end 153.19 63.8083) (width 0.2) (layer "B.Cu") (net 36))
 (segment (start 157.5 61) (end 155.9983 61) (width 0.2) (layer "B.Cu") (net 36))
 (segment (start 153.19 63.8083) (end 146.5 63.8083) (width 0.2) (layer "B.Cu") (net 36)))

